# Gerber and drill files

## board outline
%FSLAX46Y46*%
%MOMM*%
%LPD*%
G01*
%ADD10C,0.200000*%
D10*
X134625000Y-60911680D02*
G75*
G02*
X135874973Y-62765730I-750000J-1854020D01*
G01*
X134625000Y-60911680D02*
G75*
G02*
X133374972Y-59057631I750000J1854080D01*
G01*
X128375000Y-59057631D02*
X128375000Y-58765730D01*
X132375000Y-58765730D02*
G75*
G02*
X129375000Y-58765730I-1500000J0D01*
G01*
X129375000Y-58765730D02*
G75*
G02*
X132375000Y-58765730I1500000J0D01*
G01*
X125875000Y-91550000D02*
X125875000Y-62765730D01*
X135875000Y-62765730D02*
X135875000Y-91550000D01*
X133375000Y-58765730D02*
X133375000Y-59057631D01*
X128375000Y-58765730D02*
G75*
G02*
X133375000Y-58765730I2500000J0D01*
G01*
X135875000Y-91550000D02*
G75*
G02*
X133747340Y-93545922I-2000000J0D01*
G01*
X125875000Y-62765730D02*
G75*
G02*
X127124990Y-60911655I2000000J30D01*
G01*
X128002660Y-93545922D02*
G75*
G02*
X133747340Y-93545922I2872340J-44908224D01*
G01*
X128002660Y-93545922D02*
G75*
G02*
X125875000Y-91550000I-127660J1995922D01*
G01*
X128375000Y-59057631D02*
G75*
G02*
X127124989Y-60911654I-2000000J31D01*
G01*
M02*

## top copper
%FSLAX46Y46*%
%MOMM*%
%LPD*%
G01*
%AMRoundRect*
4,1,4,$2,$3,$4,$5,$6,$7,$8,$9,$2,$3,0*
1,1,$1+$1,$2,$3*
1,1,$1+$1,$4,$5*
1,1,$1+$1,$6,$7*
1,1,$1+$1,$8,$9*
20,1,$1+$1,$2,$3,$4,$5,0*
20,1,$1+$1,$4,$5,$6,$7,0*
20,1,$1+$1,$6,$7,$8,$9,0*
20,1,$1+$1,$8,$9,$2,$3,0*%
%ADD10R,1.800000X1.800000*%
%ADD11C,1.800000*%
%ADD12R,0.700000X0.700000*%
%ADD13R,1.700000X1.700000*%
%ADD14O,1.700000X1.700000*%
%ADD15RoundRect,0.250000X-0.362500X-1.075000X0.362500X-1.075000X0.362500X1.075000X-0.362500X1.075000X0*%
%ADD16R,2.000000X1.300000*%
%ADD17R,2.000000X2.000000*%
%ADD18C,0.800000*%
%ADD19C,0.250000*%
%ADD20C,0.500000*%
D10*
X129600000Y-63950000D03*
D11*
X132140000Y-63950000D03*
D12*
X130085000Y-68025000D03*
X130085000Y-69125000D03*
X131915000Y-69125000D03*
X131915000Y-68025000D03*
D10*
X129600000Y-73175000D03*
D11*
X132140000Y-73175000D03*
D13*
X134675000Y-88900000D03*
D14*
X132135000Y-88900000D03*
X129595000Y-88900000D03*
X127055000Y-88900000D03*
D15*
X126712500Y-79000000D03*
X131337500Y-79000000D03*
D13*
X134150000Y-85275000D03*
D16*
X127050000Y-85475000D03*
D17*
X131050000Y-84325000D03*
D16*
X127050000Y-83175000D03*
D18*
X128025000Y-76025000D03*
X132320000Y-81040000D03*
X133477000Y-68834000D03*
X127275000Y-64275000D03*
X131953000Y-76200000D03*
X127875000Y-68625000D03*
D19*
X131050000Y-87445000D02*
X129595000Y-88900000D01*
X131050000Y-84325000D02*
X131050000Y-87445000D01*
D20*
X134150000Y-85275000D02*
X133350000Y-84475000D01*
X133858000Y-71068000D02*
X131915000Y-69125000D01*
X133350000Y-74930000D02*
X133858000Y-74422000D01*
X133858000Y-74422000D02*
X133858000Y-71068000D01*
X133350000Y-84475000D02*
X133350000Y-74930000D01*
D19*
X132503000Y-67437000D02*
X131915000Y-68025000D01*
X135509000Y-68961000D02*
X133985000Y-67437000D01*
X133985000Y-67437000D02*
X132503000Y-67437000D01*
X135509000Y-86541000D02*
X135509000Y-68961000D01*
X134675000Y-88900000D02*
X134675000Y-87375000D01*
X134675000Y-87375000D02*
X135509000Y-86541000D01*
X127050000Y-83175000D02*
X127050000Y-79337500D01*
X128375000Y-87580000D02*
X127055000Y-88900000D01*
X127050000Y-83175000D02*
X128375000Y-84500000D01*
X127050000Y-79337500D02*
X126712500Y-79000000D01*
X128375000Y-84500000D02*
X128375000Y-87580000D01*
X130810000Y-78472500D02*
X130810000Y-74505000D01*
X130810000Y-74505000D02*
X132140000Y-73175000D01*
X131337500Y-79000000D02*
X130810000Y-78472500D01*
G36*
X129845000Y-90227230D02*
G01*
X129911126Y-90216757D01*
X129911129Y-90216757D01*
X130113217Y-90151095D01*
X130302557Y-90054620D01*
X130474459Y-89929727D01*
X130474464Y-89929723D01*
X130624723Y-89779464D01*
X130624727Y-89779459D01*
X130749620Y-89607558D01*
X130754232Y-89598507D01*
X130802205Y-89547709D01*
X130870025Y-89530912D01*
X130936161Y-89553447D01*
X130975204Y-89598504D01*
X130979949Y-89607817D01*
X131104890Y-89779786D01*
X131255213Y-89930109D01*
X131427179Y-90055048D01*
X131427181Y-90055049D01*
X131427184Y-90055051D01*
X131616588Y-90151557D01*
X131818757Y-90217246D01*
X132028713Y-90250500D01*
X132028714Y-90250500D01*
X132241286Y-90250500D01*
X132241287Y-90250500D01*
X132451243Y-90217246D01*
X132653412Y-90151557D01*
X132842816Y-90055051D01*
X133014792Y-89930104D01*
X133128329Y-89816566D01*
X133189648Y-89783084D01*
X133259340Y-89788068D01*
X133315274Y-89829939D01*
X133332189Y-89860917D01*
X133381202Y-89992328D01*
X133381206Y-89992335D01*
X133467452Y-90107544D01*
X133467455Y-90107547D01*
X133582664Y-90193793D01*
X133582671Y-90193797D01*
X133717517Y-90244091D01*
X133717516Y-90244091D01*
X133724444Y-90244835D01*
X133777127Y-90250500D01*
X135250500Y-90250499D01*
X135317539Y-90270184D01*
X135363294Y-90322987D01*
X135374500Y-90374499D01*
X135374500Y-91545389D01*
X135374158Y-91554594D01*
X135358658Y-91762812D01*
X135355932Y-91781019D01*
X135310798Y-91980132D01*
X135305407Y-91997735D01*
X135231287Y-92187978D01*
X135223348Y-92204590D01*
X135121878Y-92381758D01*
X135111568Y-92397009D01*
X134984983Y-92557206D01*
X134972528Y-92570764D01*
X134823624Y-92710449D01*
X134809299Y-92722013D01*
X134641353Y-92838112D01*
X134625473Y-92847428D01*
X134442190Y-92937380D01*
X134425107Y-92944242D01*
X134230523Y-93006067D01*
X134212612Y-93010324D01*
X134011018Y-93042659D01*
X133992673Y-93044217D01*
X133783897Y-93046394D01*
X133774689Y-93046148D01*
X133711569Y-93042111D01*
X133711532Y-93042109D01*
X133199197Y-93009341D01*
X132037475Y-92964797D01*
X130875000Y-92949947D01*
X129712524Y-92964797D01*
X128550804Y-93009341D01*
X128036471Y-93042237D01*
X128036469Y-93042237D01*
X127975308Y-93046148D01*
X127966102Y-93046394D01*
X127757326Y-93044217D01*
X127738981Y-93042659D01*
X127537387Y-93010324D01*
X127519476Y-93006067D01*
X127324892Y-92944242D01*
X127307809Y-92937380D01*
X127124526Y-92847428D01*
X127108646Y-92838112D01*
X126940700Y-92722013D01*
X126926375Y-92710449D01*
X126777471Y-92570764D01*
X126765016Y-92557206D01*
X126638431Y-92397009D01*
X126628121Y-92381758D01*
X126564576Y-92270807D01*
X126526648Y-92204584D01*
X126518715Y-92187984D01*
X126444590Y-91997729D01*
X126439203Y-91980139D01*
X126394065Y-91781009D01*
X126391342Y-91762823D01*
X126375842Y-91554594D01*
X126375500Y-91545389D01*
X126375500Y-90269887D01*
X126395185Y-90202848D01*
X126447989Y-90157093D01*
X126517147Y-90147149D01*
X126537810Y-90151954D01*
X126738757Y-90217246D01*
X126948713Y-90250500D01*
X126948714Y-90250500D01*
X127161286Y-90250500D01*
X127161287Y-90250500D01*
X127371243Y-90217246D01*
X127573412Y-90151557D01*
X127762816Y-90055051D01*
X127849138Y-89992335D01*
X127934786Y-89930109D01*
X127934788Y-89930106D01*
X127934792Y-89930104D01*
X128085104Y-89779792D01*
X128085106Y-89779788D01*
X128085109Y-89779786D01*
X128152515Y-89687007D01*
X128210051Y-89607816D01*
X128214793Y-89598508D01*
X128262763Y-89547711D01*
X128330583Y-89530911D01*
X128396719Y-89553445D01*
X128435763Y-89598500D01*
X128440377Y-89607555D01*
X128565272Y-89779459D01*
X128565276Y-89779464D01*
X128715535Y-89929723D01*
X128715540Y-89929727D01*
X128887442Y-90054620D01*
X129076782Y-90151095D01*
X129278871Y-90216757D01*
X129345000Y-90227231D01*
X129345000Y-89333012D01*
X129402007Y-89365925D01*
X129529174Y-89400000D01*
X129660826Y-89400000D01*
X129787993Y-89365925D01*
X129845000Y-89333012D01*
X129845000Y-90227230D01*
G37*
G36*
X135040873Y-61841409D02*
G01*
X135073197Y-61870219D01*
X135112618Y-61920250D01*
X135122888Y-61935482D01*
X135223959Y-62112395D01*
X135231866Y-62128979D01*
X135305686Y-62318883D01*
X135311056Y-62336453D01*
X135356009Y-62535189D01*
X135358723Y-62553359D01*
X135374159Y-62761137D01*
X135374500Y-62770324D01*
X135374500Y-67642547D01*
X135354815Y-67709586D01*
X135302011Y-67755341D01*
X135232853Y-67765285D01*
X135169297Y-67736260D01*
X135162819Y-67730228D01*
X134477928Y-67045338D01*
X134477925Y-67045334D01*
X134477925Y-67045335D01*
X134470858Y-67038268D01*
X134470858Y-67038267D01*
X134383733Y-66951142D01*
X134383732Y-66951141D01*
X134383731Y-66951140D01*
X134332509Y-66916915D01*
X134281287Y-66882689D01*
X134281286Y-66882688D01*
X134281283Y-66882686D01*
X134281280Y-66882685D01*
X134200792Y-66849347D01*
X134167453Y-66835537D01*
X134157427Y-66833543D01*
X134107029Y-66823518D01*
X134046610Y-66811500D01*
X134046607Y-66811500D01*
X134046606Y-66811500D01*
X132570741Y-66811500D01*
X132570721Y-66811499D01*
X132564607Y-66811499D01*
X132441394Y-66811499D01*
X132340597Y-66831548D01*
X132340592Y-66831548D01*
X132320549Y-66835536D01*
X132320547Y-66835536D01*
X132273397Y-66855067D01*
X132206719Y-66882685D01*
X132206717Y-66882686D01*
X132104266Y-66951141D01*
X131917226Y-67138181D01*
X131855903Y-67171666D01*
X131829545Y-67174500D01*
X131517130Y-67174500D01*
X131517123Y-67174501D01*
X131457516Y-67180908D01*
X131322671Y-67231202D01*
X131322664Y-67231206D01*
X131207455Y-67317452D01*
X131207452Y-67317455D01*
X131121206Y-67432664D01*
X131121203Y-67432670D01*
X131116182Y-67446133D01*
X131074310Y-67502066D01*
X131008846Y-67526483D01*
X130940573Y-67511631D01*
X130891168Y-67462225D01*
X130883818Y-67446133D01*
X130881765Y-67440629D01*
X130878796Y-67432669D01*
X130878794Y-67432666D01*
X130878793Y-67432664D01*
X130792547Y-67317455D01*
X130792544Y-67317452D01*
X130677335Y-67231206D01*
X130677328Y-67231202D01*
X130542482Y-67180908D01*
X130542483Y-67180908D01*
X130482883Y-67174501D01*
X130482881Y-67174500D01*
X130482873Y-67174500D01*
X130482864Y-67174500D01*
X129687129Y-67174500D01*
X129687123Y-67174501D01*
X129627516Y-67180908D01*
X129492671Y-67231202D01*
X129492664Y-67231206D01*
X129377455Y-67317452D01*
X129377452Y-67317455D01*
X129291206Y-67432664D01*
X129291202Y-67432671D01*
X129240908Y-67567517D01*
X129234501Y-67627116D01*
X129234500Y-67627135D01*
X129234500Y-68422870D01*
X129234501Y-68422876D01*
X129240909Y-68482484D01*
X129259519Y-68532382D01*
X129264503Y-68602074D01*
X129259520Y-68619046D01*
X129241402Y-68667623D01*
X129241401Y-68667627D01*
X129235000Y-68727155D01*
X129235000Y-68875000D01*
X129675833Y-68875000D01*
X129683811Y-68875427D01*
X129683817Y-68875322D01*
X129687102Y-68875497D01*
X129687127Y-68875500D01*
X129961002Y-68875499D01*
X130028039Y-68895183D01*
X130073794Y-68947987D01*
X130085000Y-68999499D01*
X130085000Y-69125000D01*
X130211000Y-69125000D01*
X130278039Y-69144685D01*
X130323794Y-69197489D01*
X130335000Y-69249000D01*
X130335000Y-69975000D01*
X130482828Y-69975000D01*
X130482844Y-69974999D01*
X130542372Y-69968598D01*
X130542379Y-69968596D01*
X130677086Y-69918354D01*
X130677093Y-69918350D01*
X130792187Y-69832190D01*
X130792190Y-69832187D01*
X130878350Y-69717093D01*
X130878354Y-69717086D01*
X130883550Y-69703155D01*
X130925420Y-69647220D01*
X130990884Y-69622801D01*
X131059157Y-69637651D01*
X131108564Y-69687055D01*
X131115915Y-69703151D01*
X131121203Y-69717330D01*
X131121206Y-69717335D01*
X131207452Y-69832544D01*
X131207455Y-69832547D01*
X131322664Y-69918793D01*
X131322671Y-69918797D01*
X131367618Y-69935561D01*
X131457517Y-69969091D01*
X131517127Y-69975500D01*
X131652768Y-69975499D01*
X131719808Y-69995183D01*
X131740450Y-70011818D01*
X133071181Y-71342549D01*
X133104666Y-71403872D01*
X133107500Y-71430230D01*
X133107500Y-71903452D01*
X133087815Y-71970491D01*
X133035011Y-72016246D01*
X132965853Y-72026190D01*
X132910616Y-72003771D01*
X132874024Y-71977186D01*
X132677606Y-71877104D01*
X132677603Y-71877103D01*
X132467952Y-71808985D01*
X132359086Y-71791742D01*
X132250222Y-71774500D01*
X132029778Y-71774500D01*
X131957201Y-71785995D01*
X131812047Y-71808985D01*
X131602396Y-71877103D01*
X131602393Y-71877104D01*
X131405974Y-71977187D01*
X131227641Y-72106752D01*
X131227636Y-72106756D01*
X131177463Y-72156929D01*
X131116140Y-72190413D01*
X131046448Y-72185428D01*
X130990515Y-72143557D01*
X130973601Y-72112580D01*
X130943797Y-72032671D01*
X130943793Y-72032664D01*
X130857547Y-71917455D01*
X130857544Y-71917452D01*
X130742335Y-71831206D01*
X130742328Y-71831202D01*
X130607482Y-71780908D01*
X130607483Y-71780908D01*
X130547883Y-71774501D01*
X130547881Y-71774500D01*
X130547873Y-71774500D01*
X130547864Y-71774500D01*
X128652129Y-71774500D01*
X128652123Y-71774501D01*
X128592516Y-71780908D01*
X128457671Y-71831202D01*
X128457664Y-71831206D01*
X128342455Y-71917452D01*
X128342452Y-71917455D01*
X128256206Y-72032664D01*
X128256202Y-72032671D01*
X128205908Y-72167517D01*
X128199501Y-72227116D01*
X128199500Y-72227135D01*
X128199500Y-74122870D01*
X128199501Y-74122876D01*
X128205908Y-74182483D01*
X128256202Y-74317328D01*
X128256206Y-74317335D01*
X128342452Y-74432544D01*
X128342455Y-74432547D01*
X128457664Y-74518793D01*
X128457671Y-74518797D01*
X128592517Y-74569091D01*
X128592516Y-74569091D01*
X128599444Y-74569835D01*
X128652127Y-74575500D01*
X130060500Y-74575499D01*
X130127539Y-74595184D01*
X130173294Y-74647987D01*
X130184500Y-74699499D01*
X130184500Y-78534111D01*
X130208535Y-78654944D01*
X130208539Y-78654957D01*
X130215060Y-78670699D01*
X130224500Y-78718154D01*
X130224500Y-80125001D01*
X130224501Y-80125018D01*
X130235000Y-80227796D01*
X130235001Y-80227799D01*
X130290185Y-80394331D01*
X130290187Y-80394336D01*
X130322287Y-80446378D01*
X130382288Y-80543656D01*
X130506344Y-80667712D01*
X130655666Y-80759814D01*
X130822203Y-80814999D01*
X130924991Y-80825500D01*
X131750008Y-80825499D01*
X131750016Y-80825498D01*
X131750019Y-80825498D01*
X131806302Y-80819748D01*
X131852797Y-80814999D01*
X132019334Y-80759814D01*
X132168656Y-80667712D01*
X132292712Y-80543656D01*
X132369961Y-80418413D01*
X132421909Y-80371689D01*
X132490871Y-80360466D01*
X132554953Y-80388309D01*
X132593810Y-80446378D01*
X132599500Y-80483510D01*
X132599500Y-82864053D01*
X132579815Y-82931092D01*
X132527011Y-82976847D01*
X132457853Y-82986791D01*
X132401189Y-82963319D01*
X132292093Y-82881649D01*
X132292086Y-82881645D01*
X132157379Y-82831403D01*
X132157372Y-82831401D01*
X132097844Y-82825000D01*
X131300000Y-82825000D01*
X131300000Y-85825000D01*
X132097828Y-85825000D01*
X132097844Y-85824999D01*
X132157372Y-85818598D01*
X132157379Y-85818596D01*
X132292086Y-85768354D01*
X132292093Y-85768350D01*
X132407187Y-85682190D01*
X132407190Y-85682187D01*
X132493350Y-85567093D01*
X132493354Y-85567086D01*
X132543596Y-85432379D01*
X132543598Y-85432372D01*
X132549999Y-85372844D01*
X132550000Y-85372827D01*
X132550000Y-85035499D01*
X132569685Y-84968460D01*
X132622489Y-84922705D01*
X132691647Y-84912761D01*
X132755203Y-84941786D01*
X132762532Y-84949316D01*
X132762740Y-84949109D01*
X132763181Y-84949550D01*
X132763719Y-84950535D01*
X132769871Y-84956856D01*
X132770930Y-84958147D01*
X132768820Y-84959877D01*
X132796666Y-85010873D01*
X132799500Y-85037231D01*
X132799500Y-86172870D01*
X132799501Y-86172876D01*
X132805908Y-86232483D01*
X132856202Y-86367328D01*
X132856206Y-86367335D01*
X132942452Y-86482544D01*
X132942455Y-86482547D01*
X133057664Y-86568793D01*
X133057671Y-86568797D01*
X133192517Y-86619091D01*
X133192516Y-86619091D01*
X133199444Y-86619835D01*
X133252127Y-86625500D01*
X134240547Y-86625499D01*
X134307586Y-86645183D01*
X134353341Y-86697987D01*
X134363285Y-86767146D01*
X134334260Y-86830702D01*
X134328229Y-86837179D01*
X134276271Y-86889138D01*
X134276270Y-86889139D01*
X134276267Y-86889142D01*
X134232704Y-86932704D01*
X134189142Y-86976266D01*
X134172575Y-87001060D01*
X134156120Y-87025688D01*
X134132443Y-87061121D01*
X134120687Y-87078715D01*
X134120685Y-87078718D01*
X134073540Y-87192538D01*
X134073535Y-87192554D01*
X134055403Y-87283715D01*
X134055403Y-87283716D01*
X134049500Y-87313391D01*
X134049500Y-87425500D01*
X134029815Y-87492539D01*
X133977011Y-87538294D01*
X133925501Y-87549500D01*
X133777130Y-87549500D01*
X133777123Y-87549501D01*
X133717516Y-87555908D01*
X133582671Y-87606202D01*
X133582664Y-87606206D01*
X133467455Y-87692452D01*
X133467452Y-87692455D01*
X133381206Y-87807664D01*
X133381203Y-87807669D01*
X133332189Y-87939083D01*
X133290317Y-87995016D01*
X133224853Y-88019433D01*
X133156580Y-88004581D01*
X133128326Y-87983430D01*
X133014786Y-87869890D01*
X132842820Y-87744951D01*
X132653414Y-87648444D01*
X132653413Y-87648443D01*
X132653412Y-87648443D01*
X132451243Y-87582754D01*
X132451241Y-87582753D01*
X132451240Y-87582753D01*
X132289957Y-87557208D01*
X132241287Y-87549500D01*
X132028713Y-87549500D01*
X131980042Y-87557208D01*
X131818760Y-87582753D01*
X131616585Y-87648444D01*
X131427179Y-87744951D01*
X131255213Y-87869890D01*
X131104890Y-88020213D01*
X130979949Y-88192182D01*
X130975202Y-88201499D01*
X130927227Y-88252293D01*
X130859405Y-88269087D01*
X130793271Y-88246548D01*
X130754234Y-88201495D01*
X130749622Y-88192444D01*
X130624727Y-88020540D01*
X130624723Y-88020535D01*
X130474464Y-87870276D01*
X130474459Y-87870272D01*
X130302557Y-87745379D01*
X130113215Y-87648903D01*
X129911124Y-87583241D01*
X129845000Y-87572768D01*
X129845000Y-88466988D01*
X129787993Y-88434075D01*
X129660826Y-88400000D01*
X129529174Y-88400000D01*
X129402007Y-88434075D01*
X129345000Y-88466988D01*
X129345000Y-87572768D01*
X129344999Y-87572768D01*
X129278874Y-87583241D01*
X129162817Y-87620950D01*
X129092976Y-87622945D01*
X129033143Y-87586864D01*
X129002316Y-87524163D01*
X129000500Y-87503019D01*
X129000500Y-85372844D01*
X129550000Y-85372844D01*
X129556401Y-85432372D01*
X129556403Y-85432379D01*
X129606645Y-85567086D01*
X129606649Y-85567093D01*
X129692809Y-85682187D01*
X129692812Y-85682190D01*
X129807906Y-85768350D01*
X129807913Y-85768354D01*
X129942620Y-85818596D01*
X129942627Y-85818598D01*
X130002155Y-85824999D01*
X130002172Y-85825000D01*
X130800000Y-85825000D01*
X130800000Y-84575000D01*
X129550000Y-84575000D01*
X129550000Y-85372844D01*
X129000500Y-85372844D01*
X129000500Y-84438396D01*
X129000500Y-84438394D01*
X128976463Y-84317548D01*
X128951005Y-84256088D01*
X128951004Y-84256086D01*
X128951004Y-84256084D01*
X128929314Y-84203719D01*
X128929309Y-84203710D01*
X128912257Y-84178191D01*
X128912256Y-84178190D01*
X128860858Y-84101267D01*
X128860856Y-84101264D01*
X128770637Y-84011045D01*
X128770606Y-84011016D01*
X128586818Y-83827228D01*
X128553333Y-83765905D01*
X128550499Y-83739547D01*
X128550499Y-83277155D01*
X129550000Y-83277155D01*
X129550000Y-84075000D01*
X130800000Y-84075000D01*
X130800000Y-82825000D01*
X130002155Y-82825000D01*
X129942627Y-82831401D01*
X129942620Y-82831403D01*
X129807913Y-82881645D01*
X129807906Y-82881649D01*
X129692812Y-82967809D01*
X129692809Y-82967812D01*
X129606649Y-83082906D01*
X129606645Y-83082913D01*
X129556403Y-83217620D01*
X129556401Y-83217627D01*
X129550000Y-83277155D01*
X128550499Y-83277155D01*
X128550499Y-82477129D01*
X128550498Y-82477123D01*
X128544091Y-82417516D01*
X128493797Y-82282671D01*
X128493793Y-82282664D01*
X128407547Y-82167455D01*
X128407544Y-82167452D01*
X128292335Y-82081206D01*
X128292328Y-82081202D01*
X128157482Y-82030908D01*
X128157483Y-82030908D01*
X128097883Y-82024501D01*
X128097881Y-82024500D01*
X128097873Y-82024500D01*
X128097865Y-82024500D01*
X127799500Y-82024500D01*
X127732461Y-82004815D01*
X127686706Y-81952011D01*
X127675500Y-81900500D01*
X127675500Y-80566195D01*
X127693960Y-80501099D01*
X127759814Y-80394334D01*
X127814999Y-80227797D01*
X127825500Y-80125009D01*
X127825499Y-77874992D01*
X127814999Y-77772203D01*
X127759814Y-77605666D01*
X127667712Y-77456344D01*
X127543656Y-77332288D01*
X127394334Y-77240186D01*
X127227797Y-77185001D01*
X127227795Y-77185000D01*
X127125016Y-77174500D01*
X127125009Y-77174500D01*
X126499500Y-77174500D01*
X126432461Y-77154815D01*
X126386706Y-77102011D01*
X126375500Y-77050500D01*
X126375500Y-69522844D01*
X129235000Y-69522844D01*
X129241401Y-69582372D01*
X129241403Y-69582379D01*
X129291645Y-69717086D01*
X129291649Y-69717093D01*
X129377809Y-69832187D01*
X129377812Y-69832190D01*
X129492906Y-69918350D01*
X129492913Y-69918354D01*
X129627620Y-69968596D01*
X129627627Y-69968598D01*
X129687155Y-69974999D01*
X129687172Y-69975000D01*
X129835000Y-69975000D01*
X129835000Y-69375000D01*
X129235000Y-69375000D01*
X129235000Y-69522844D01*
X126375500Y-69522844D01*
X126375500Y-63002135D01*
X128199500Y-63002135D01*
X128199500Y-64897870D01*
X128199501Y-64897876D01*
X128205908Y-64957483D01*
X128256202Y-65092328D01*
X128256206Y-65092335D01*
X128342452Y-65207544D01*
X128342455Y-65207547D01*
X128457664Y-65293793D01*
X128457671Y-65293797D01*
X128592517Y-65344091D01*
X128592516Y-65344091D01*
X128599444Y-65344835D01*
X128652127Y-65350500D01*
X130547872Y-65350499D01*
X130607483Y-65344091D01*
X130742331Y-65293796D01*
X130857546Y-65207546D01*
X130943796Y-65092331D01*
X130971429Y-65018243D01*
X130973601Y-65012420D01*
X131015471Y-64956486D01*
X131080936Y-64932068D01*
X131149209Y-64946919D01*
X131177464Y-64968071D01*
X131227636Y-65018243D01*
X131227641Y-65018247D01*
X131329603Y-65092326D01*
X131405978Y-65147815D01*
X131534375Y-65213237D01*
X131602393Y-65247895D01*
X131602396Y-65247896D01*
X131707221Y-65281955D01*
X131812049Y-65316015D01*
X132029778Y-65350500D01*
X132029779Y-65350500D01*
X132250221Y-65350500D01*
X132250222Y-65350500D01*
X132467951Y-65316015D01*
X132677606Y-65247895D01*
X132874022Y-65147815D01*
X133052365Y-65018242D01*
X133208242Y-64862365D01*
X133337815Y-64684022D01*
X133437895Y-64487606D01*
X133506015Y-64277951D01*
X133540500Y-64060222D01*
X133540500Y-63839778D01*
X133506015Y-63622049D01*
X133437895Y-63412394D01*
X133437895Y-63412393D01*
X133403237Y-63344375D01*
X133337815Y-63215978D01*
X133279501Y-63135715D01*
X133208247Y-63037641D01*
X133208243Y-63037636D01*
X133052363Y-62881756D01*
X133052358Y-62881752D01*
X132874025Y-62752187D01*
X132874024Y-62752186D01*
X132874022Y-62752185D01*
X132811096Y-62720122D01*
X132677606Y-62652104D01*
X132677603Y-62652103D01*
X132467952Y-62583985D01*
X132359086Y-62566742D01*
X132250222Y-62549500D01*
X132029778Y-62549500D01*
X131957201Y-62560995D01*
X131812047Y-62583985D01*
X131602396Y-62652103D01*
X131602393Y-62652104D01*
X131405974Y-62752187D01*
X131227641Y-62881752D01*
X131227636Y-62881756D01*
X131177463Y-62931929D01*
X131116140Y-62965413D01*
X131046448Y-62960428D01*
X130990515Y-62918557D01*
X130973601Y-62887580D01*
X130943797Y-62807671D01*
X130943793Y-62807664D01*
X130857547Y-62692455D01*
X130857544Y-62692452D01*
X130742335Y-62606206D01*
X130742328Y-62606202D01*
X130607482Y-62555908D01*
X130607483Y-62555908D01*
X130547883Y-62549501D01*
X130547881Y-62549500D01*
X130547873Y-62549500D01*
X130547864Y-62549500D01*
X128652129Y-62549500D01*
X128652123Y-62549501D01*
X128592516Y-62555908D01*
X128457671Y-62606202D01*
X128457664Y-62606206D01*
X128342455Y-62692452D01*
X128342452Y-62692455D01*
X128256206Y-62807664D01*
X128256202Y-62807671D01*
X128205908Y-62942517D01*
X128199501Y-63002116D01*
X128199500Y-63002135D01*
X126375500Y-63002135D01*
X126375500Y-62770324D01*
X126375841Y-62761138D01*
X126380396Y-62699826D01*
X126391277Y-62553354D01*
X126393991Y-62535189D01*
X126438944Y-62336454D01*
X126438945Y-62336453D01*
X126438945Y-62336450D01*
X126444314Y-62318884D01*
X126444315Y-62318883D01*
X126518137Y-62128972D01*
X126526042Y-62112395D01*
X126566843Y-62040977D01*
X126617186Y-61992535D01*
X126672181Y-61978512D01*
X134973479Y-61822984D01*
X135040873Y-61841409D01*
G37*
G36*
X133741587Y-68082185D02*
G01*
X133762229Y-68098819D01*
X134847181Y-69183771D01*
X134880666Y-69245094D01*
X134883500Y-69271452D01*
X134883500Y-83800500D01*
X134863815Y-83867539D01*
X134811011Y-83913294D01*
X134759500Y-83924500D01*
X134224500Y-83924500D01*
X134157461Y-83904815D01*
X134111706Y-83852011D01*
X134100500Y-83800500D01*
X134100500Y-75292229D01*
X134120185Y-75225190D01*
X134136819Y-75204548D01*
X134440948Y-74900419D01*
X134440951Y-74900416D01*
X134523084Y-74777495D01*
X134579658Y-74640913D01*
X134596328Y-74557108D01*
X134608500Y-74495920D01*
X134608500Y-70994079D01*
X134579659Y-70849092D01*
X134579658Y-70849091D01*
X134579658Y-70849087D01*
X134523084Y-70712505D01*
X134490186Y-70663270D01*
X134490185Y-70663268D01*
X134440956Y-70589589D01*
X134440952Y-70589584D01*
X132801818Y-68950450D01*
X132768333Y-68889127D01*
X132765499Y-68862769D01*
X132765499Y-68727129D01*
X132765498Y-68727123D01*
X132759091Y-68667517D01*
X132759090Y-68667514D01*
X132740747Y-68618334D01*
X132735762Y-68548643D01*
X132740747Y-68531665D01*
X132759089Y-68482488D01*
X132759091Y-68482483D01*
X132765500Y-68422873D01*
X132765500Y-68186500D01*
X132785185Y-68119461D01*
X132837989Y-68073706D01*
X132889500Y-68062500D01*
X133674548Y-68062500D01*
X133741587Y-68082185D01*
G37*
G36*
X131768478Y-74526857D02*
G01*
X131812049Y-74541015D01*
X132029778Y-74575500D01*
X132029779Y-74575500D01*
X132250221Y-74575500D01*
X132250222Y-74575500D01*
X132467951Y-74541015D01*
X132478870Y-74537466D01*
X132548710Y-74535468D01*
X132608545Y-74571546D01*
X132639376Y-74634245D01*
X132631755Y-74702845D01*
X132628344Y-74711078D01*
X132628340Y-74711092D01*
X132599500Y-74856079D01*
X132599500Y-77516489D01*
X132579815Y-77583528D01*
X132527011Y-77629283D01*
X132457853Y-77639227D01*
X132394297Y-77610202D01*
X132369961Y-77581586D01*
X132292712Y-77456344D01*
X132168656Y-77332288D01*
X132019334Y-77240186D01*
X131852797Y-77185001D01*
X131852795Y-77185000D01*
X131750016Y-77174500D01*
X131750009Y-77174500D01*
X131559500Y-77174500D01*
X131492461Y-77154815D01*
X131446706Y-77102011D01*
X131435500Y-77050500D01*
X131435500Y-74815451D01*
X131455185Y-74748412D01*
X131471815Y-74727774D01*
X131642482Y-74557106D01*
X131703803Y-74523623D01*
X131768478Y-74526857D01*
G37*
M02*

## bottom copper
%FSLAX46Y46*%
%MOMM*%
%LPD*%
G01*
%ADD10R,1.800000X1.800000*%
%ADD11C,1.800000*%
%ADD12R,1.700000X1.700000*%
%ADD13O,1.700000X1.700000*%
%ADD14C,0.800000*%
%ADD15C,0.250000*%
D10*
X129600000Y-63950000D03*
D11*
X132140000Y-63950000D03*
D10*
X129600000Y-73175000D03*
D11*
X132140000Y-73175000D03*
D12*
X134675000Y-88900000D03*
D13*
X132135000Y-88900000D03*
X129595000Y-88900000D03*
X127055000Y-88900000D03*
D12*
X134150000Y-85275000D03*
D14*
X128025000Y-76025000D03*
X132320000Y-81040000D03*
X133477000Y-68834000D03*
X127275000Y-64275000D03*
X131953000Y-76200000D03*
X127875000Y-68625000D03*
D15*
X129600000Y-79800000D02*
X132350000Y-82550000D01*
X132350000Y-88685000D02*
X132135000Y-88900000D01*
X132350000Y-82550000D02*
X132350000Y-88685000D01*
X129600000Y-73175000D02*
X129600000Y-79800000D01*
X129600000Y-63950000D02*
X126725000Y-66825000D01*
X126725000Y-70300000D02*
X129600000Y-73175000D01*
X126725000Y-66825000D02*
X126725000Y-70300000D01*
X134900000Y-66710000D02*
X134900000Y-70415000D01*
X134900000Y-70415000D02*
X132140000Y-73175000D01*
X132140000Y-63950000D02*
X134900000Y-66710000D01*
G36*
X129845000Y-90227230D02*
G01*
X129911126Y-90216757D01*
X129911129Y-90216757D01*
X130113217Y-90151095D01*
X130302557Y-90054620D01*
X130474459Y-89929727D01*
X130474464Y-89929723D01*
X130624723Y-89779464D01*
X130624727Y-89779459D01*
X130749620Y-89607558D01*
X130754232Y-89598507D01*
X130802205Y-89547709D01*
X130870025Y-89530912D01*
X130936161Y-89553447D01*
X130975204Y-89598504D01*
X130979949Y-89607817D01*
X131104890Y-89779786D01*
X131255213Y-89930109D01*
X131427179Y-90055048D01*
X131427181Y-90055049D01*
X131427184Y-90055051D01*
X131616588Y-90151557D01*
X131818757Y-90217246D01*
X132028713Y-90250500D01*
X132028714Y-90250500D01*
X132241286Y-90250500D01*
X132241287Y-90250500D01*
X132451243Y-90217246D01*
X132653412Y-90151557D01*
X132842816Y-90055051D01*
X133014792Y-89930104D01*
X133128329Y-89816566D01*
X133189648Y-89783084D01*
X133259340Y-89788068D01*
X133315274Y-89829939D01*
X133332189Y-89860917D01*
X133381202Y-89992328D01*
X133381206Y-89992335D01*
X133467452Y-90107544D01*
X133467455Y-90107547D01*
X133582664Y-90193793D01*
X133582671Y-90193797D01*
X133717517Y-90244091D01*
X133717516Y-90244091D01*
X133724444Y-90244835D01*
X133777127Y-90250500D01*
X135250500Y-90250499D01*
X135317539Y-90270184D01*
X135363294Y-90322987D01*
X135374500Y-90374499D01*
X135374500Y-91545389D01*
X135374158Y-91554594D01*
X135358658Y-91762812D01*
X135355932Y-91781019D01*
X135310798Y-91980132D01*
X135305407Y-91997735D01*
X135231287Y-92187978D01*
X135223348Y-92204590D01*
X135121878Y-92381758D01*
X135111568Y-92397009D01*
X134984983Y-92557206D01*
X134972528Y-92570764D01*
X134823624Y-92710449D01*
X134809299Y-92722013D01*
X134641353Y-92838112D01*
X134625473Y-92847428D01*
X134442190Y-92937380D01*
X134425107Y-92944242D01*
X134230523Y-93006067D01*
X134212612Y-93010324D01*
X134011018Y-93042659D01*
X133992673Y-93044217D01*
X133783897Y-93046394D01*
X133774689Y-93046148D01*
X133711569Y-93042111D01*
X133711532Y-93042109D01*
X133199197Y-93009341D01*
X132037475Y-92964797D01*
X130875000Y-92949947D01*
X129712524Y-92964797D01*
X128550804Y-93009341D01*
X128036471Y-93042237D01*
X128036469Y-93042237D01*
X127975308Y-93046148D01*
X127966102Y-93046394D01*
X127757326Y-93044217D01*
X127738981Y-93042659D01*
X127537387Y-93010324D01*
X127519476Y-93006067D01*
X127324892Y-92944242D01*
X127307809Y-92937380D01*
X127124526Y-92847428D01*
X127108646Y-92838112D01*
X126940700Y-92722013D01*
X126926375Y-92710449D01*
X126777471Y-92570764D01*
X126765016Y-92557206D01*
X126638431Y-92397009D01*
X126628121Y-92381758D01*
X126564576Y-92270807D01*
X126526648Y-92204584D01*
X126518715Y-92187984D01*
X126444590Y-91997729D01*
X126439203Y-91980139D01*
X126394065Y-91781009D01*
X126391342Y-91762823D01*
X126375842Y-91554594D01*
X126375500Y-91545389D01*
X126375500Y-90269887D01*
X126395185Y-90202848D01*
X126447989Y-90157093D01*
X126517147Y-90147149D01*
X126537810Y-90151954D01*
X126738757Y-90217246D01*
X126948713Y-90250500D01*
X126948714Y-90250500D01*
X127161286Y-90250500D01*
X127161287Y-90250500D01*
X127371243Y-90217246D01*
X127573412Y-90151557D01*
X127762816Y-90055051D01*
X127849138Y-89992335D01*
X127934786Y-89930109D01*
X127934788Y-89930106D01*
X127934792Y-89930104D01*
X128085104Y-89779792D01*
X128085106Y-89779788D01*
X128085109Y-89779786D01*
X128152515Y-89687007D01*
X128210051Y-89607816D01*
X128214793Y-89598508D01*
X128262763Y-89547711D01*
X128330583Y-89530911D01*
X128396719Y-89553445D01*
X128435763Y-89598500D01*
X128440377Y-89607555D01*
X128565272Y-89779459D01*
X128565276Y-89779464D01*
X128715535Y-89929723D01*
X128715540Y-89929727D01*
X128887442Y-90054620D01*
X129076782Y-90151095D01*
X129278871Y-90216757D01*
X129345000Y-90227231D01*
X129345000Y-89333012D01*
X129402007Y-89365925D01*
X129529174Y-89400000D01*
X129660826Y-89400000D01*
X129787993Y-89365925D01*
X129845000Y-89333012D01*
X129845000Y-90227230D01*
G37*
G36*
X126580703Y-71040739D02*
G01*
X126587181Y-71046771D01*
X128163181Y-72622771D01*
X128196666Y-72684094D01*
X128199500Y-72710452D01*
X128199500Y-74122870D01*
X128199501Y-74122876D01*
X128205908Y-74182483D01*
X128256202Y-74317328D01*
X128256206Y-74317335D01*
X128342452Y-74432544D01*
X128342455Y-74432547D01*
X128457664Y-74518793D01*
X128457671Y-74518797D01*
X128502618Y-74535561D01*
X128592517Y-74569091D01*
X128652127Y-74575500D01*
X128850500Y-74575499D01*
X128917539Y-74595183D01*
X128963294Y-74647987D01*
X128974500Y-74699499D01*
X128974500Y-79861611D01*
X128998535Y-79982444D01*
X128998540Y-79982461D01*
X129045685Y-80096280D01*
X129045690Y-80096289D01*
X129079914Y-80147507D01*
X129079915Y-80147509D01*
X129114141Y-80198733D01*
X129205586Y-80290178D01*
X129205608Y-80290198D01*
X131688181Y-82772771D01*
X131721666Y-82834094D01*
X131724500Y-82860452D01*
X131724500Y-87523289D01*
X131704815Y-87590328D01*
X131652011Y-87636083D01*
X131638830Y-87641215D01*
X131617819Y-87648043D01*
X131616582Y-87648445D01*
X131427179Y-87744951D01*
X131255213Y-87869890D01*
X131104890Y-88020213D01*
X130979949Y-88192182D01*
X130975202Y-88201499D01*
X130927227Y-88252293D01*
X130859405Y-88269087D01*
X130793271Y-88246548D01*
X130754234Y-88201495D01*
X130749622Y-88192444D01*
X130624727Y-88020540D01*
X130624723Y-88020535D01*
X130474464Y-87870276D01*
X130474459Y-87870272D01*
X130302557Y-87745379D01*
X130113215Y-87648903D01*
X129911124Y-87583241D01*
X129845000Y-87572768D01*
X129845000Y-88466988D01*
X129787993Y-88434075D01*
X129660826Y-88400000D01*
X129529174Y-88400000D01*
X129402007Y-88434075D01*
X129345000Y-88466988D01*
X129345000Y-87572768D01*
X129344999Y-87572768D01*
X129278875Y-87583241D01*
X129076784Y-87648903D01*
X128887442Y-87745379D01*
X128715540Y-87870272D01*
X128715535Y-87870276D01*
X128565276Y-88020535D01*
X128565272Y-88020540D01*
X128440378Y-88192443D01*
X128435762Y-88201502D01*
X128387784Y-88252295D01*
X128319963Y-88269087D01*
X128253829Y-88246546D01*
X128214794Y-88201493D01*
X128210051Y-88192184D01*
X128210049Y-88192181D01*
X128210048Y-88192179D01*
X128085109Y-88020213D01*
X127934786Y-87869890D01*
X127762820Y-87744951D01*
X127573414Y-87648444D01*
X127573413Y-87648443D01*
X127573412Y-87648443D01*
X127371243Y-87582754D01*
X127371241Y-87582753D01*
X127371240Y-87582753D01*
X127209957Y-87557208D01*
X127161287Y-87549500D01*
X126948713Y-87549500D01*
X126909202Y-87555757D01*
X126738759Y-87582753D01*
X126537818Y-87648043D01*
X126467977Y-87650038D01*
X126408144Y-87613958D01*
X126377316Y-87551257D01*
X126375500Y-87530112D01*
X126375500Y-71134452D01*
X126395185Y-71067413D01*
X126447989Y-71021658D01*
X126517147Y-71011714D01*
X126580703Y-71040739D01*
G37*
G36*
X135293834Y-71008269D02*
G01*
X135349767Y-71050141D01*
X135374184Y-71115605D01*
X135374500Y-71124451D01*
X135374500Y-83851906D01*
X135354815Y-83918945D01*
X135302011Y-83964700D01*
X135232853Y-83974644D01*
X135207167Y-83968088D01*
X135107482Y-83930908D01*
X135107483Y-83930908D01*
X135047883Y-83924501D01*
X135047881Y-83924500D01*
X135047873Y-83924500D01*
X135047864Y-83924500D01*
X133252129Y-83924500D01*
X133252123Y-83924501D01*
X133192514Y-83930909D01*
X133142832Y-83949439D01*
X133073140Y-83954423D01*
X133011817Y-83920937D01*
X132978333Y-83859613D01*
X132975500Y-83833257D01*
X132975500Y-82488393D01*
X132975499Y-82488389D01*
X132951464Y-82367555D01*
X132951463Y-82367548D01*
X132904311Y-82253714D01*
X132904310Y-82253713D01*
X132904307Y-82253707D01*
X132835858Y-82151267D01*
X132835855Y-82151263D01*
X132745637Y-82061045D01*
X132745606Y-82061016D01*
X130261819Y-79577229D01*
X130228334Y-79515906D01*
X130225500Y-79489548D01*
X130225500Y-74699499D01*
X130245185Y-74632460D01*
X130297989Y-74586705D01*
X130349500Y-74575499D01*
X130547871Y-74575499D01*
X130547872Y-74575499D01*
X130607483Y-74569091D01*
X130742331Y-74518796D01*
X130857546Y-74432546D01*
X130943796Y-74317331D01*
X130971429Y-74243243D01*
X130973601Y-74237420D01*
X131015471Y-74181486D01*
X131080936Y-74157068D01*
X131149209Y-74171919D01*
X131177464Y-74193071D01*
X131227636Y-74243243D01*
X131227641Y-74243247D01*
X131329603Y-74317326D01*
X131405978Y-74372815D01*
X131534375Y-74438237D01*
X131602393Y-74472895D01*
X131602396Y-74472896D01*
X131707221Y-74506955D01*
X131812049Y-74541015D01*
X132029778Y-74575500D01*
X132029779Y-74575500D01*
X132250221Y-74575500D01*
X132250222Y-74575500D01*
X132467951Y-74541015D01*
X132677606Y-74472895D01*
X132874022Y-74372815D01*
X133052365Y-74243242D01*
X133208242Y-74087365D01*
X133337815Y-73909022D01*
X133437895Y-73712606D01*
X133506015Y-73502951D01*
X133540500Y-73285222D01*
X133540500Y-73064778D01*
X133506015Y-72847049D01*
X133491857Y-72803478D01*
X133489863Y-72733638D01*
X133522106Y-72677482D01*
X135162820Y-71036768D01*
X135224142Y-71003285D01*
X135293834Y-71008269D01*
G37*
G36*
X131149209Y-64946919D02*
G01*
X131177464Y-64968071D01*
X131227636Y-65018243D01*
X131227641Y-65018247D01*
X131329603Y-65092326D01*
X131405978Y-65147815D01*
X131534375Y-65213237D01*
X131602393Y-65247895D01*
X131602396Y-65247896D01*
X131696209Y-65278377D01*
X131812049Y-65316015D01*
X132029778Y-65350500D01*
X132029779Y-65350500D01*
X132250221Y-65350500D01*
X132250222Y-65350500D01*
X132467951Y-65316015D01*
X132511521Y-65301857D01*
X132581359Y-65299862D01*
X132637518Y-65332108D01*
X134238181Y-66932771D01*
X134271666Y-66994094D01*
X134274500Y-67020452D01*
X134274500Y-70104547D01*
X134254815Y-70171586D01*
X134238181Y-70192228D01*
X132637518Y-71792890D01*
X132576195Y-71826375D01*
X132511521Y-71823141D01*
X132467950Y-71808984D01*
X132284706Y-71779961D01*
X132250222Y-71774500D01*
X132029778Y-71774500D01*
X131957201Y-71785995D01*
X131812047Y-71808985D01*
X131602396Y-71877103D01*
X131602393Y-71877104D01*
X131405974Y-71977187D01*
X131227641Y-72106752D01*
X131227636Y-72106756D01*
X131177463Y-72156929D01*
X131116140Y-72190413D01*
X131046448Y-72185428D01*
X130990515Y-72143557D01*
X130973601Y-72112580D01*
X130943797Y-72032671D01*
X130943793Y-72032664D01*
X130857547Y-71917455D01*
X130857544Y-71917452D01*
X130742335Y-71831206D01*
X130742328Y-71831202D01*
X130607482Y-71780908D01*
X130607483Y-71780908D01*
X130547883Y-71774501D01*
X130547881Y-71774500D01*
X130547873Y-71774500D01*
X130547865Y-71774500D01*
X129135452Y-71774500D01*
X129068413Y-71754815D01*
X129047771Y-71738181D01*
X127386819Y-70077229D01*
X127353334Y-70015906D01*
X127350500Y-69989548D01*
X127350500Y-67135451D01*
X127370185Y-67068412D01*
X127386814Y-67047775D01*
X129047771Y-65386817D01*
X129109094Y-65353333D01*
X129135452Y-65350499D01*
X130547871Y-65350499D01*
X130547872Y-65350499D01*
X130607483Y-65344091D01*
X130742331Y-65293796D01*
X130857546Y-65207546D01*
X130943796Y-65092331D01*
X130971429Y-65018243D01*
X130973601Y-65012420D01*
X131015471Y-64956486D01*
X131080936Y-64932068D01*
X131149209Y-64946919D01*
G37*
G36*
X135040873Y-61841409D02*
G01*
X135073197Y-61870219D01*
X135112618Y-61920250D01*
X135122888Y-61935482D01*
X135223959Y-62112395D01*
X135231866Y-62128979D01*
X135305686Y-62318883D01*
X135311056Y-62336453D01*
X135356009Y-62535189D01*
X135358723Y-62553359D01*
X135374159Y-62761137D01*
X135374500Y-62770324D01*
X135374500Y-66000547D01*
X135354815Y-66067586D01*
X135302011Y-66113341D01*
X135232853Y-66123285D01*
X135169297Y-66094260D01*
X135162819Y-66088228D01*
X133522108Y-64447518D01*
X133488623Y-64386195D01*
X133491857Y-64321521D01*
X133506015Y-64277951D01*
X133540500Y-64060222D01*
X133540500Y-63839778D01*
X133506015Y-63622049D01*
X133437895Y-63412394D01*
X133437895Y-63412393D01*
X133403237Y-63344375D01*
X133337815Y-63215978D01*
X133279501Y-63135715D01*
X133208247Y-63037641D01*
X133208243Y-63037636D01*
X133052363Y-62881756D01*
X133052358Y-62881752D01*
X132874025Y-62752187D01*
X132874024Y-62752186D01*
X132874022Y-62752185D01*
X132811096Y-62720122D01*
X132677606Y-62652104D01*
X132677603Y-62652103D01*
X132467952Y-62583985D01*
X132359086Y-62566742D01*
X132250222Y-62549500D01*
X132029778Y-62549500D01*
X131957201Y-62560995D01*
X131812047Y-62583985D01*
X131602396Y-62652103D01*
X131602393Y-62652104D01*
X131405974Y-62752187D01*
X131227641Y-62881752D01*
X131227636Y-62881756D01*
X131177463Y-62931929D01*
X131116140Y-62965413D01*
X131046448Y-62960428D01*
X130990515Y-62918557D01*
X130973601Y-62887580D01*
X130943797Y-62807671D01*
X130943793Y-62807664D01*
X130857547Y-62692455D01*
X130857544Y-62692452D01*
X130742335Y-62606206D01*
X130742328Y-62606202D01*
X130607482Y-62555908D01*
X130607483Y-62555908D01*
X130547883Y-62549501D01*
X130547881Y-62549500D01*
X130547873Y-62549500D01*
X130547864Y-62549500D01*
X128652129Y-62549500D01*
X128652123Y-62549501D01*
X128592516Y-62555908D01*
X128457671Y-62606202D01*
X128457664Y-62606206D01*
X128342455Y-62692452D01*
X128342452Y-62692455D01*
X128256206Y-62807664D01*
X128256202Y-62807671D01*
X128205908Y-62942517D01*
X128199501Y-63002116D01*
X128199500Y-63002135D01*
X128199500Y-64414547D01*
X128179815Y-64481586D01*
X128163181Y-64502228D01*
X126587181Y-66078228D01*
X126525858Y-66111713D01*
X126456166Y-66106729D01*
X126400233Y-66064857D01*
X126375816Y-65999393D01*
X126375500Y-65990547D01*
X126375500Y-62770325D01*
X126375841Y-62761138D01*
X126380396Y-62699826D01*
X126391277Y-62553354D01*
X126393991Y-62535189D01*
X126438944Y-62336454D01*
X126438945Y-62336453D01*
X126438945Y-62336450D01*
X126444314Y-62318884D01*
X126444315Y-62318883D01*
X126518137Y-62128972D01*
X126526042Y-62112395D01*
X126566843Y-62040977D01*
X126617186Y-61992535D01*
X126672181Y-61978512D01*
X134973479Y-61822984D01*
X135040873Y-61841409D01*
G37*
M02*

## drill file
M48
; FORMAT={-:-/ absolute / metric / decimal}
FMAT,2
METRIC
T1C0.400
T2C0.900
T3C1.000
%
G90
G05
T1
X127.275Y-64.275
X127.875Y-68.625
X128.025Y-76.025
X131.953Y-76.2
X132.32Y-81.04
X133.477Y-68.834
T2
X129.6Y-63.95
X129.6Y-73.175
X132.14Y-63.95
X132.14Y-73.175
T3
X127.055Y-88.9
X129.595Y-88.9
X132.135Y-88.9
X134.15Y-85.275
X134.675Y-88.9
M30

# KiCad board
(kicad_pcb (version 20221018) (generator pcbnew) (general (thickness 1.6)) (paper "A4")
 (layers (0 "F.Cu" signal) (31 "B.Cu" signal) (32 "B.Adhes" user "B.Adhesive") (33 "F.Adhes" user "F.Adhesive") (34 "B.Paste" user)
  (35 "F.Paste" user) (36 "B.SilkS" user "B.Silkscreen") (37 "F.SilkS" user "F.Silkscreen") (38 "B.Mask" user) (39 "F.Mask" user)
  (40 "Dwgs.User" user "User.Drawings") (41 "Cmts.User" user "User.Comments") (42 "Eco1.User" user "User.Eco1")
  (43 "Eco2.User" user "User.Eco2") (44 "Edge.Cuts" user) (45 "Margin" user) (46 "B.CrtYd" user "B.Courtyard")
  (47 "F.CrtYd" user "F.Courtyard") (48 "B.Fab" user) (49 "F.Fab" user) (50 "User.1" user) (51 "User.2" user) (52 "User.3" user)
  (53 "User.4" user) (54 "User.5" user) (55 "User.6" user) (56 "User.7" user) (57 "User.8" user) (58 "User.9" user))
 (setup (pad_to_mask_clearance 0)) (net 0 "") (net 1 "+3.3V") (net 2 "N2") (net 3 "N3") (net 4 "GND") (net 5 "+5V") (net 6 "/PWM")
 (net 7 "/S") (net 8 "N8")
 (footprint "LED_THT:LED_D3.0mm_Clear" (layer "F.Cu") (at 129.6 63.95)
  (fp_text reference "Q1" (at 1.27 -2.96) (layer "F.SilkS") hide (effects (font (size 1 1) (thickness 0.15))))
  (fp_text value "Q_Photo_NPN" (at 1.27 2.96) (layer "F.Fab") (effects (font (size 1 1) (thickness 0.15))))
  (pad "1" thru_hole rect (at 0 0) (size 1.8 1.8) (drill 0.9) (layers "*.Cu" "*.Mask") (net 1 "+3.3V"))
  (pad "2" thru_hole circle (at 2.54 0) (size 1.8 1.8) (drill 0.9) (layers "*.Cu" "*.Mask") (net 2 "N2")))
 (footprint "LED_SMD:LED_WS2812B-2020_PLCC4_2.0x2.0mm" (layer "F.Cu") (at 131 68.575)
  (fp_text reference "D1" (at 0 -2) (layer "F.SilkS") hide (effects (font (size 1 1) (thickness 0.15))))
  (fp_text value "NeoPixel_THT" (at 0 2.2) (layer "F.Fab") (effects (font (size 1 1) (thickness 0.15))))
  (pad "1" smd rect (at -0.915 -0.55) (size 0.7 0.7) (layers "F.Cu" "F.Paste" "F.Mask") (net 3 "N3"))
  (pad "2" smd rect (at -0.915 0.55) (size 0.7 0.7) (layers "F.Cu" "F.Paste" "F.Mask") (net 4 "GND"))
  (pad "3" smd rect (at 0.915 0.55) (size 0.7 0.7) (layers "F.Cu" "F.Paste" "F.Mask") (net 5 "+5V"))
  (pad "4" smd rect (at 0.915 -0.55) (size 0.7 0.7) (layers "F.Cu" "F.Paste" "F.Mask") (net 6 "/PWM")))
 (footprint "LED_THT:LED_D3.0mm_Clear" (layer "F.Cu") (at 129.6 73.175)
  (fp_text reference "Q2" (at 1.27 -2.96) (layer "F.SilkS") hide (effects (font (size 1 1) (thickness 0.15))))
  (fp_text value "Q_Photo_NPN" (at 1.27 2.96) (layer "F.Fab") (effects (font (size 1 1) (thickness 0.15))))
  (pad "1" thru_hole rect (at 0 0) (size 1.8 1.8) (drill 0.9) (layers "*.Cu" "*.Mask") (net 1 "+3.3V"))
  (pad "2" thru_hole circle (at 2.54 0) (size 1.8 1.8) (drill 0.9) (layers "*.Cu" "*.Mask") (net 2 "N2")))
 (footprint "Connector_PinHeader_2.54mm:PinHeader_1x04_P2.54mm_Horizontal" (layer "F.Cu") (at 134.675 88.9 -90)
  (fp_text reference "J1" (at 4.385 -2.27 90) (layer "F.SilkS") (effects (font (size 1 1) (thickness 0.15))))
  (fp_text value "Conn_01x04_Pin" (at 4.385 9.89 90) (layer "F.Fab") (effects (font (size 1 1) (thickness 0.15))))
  (pad "1" thru_hole rect (at 0 0 270) (size 1.7 1.7) (drill 1) (layers "*.Cu" "*.Mask") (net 6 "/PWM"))
  (pad "2" thru_hole oval (at 0 2.54 270) (size 1.7 1.7) (drill 1) (layers "*.Cu" "*.Mask") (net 1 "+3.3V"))
  (pad "3" thru_hole oval (at 0 5.08 270) (size 1.7 1.7) (drill 1) (layers "*.Cu" "*.Mask") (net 4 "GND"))
  (pad "4" thru_hole oval (at 0 7.62 270) (size 1.7 1.7) (drill 1) (layers "*.Cu" "*.Mask") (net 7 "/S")))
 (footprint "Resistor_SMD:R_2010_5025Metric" (layer "F.Cu") (at 129.025 79)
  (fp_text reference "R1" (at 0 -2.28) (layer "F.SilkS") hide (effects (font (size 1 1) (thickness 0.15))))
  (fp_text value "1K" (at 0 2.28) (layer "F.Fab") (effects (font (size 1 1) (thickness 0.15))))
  (pad "1" smd roundrect (at -2.3125 0) (size 1.225 2.65) (layers "F.Cu" "F.Paste" "F.Mask") (roundrect_rratio 0.2040816327) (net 7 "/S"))
  (pad "2" smd roundrect (at 2.3125 0) (size 1.225 2.65) (layers "F.Cu" "F.Paste" "F.Mask") (roundrect_rratio 0.2040816327) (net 2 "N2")))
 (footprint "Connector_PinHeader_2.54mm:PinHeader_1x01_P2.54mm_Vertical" (layer "F.Cu") (at 134.15 85.275)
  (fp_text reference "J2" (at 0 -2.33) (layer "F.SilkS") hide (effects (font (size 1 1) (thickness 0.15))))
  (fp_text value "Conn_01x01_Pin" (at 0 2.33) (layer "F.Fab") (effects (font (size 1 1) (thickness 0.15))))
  (pad "1" thru_hole rect (at 0 0) (size 1.7 1.7) (drill 1) (layers "*.Cu" "*.Mask") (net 5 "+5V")))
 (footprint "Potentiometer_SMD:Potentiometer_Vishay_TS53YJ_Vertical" (layer "F.Cu") (at 129.05 84.325 180)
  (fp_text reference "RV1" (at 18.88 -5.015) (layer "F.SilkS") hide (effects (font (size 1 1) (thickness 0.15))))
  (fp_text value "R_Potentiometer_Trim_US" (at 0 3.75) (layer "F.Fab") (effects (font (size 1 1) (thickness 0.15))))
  (pad "1" smd rect (at 2 -1.15 180) (size 2 1.3) (layers "F.Cu" "F.Paste" "F.Mask") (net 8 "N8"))
  (pad "2" smd rect (at -2 0 180) (size 2 2) (layers "F.Cu" "F.Paste" "F.Mask") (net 4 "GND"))
  (pad "3" smd rect (at 2 1.15 180) (size 2 1.3) (layers "F.Cu" "F.Paste" "F.Mask") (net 7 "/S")))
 (gr_arc (start 134.625 60.91168) (mid 135.533312 61.647696) (end 135.875 62.76573) (stroke (width 0.2) (type solid)) (layer "Edge.Cuts"))
 (gr_arc (start 134.625 60.91168) (mid 133.716688 60.175665) (end 133.375 59.057631) (stroke (width 0.2) (type solid)) (layer "Edge.Cuts"))
 (gr_line (start 128.375 59.057631) (end 128.375 58.76573) (stroke (width 0.2) (type solid)) (layer "Edge.Cuts"))
 (gr_circle (center 130.875 58.76573) (end 129.375 58.76573) (stroke (width 0.2) (type solid)) (fill none) (layer "Edge.Cuts"))
 (gr_line (start 125.875 91.55) (end 125.875 62.76573) (stroke (width 0.2) (type solid)) (layer "Edge.Cuts"))
 (gr_line (start 135.875 62.76573) (end 135.875 91.55) (stroke (width 0.2) (type solid)) (layer "Edge.Cuts"))
 (gr_line (start 133.375 58.76573) (end 133.375 59.057631) (stroke (width 0.2) (type solid)) (layer "Edge.Cuts"))
 (gr_arc (start 128.375 58.76573) (mid 130.875 56.26573) (end 133.375 58.76573) (stroke (width 0.2) (type solid)) (layer "Edge.Cuts"))
 (gr_arc (start 135.875 91.55) (mid 135.243335 93.00865) (end 133.74734 93.545922) (stroke (width 0.2) (type solid)) (layer "Edge.Cuts"))
 (gr_arc (start 125.875 62.76573) (mid 126.216689 61.647697) (end 127.125 60.91168) (stroke (width 0.2) (type solid)) (layer "Edge.Cuts"))
 (gr_arc (start 128.00266 93.545922) (mid 130.875 93.454158) (end 133.74734 93.545922) (stroke (width 0.2) (type solid)) (layer "Edge.Cuts"))
 (gr_arc (start 128.00266 93.545922) (mid 126.506665 93.00865) (end 125.875 91.55) (stroke (width 0.2) (type solid)) (layer "Edge.Cuts"))
 (gr_arc (start 128.375 59.057631) (mid 128.033313 60.175666) (end 127.125 60.91168) (stroke (width 0.2) (type solid)) (layer "Edge.Cuts"))
 (segment (start 131.05 87.445) (end 129.595 88.9) (width 0.25) (layer "F.Cu") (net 4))
 (segment (start 131.05 84.325) (end 131.05 87.445) (width 0.25) (layer "F.Cu") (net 4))
 (via (at 128.025 76.025) (size 0.8) (drill 0.4) (layers "F.Cu" "B.Cu") (free) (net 4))
 (via (at 132.32 81.04) (size 0.8) (drill 0.4) (layers "F.Cu" "B.Cu") (free) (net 4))
 (via (at 133.477 68.834) (size 0.8) (drill 0.4) (layers "F.Cu" "B.Cu") (free) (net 4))
 (via (at 127.275 64.275) (size 0.8) (drill 0.4) (layers "F.Cu" "B.Cu") (free) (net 4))
 (via (at 131.953 76.2) (size 0.8) (drill 0.4) (layers "F.Cu" "B.Cu") (free) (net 4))
 (via (at 127.875 68.625) (size 0.8) (drill 0.4) (layers "F.Cu" "B.Cu") (free) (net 4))
 (segment (start 134.15 85.275) (end 133.35 84.475) (width 0.5) (layer "F.Cu") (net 5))
 (segment (start 133.858 71.068) (end 131.915 69.125) (width 0.5) (layer "F.Cu") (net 5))
 (segment (start 133.35 74.93) (end 133.858 74.422) (width 0.5) (layer "F.Cu") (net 5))
 (segment (start 133.858 74.422) (end 133.858 71.068) (width 0.5) (layer "F.Cu") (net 5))
 (segment (start 133.35 84.475) (end 133.35 74.93) (width 0.5) (layer "F.Cu") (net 5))
 (segment (start 132.503 67.437) (end 131.915 68.025) (width 0.25) (layer "F.Cu") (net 6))
 (segment (start 135.509 68.961) (end 133.985 67.437) (width 0.25) (layer "F.Cu") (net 6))
 (segment (start 133.985 67.437) (end 132.503 67.437) (width 0.25) (layer "F.Cu") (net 6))
 (segment (start 135.509 86.541) (end 135.509 68.961) (width 0.25) (layer "F.Cu") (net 6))
 (segment (start 134.675 88.9) (end 134.675 87.375) (width 0.25) (layer "F.Cu") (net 6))
 (segment (start 134.675 87.375) (end 135.509 86.541) (width 0.25) (layer "F.Cu") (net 6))
 (segment (start 129.6 79.8) (end 132.35 82.55) (width 0.25) (layer "B.Cu") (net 1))
 (segment (start 132.35 88.685) (end 132.135 88.9) (width 0.25) (layer "B.Cu") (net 1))
 (segment (start 132.35 82.55) (end 132.35 88.685) (width 0.25) (layer "B.Cu") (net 1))
 (segment (start 129.6 73.175) (end 129.6 79.8) (width 0.25) (layer "B.Cu") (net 1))
 (segment (start 129.6 63.95) (end 126.725 66.825) (width 0.25) (layer "B.Cu") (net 1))
 (segment (start 126.725 70.3) (end 129.6 73.175) (width 0.25) (layer "B.Cu") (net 1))
 (segment (start 126.725 66.825) (end 126.725 70.3) (width 0.25) (layer "B.Cu") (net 1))
 (segment (start 127.05 83.175) (end 127.05 79.3375) (width 0.25) (layer "F.Cu") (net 7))
 (segment (start 128.375 87.58) (end 127.055 88.9) (width 0.25) (layer "F.Cu") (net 7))
 (segment (start 127.05 83.175) (end 128.375 84.5) (width 0.25) (layer "F.Cu") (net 7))
 (segment (start 127.05 79.3375) (end 126.7125 79) (width 0.25) (layer "F.Cu") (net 7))
 (segment (start 128.375 84.5) (end 128.375 87.58) (width 0.25) (layer "F.Cu") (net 7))
 (segment (start 130.81 78.4725) (end 130.81 74.505) (width 0.25) (layer "F.Cu") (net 2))
 (segment (start 130.81 74.505) (end 132.14 73.175) (width 0.25) (layer "F.Cu") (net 2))
 (segment (start 131.3375 79) (end 130.81 78.4725) (width 0.25) (layer "F.Cu") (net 2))
 (segment (start 134.9 66.71) (end 134.9 70.415) (width 0.25) (layer "B.Cu") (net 2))
 (segment (start 134.9 70.415) (end 132.14 73.175) (width 0.25) (layer "B.Cu") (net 2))
 (segment (start 132.14 63.95) (end 134.9 66.71) (width 0.25) (layer "B.Cu") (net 2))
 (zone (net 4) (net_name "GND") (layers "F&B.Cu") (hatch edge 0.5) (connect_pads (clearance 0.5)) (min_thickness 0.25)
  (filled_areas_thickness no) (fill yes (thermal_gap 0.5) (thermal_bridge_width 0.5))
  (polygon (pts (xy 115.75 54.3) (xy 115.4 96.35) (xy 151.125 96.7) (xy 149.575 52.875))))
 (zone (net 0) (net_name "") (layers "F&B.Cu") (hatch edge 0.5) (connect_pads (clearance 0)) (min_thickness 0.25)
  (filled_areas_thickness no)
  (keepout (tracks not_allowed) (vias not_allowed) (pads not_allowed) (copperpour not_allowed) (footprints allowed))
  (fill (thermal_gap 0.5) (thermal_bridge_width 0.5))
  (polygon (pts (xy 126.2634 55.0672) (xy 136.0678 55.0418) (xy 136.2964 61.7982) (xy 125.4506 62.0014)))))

